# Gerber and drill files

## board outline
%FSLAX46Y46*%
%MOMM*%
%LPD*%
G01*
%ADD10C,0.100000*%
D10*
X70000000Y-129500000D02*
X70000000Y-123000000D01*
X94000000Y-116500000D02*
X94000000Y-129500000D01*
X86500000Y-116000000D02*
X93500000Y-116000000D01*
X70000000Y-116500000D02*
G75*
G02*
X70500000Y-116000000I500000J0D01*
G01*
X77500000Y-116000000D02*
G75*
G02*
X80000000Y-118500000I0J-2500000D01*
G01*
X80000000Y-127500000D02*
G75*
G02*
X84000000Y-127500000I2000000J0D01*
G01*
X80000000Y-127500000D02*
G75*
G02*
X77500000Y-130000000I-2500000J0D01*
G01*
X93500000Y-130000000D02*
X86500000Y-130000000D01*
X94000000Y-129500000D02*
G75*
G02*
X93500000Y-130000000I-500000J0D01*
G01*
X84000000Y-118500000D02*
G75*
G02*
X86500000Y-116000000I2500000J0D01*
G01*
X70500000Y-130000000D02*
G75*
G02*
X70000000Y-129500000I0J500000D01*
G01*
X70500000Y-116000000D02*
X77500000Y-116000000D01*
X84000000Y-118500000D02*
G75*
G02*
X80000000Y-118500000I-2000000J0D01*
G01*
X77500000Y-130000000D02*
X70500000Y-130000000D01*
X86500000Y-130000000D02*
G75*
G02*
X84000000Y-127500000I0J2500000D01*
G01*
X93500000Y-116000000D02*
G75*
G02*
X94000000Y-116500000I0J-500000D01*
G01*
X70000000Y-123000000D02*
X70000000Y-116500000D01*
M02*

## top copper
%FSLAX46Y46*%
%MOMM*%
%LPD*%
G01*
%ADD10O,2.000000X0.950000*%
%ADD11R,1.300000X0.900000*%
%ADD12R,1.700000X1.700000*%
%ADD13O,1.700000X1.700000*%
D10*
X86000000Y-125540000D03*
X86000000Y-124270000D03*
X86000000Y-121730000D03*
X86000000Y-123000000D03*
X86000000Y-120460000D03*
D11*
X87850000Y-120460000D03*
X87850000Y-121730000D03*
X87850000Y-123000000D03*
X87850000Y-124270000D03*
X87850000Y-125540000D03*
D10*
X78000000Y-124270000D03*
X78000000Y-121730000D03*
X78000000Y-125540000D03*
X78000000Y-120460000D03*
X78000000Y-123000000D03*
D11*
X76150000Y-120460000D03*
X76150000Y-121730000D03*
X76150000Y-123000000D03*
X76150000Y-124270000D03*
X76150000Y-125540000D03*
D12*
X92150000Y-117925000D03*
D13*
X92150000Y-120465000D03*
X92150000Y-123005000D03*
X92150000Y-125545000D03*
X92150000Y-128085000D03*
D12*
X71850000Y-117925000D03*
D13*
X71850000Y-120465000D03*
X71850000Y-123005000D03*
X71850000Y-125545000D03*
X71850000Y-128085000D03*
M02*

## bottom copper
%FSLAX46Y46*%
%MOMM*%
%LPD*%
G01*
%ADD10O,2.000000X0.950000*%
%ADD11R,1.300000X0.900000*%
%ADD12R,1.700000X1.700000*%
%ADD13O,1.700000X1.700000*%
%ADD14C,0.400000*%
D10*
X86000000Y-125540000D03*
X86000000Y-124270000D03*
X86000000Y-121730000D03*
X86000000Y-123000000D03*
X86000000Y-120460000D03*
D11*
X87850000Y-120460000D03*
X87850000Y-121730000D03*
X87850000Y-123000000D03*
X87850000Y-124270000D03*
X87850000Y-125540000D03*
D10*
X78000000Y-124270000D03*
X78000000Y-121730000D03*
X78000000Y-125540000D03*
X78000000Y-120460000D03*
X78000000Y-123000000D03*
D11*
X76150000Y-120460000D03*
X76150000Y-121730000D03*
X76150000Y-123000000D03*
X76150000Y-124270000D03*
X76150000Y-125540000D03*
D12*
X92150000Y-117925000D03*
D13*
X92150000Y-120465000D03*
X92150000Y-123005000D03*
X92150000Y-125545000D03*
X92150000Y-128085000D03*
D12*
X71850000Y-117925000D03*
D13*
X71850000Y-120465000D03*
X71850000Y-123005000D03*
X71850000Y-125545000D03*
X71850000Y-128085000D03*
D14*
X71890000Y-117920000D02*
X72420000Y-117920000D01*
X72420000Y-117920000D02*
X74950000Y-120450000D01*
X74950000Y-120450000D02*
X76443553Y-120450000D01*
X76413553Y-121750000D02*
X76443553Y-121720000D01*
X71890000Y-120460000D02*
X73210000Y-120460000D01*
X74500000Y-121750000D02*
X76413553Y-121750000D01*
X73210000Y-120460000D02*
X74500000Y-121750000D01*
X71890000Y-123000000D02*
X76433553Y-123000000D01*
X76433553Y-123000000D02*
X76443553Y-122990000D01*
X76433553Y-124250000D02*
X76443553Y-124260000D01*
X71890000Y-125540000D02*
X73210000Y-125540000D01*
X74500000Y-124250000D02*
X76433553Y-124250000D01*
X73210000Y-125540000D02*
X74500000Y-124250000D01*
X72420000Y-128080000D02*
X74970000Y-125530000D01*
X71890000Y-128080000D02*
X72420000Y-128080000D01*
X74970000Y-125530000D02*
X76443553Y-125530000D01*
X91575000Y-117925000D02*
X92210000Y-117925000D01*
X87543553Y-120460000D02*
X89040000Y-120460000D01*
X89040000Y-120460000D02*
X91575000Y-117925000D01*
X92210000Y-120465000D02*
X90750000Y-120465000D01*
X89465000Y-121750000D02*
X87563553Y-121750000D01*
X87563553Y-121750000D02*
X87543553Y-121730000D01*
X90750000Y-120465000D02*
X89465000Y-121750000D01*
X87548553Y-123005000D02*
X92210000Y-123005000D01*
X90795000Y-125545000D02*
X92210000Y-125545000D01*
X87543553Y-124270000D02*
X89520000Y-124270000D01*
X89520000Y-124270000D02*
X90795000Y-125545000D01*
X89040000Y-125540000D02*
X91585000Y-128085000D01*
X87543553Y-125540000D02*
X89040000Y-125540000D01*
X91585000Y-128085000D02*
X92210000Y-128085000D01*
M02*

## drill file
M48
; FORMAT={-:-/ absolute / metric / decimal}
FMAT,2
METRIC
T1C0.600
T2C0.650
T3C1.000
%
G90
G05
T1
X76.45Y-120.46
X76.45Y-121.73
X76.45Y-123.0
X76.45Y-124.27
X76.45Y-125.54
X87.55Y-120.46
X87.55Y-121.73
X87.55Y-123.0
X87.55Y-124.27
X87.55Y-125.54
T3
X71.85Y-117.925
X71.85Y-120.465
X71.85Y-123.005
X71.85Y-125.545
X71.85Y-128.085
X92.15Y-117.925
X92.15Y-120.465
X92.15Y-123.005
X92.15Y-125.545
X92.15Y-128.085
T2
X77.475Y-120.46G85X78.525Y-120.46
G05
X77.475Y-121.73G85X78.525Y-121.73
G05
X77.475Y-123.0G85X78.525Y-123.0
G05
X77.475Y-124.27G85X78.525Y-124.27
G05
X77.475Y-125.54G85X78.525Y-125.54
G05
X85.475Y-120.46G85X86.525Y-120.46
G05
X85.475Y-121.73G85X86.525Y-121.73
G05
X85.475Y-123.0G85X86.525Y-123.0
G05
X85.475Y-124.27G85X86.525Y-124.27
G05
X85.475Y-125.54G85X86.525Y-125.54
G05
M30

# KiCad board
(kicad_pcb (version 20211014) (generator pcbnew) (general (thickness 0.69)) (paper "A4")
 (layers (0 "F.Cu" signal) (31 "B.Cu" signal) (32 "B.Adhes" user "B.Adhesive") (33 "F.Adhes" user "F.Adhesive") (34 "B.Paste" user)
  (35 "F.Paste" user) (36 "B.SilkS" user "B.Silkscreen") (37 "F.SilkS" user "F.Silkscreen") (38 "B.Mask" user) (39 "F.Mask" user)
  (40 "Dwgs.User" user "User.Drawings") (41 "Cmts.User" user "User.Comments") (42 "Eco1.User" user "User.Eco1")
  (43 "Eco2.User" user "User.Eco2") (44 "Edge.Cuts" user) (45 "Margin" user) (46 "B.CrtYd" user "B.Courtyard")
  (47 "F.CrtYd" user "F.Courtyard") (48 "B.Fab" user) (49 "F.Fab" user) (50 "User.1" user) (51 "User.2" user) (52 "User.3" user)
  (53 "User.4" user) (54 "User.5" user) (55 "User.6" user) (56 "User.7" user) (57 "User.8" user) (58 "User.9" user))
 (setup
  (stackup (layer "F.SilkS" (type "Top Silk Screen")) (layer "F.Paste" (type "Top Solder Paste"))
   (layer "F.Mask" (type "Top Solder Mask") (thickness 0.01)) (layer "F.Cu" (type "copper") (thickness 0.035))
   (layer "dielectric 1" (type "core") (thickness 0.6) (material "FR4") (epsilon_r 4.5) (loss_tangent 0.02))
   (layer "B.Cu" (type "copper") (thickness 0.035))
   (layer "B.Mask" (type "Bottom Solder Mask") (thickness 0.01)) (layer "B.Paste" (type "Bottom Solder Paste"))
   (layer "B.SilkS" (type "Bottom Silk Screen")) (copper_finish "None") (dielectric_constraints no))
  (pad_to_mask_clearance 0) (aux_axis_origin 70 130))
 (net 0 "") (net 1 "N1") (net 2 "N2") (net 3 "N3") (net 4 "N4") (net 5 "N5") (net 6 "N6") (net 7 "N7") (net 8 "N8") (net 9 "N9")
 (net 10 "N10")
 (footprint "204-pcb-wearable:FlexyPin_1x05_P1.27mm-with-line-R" (layer "F.Cu") (at 86.05 120.46)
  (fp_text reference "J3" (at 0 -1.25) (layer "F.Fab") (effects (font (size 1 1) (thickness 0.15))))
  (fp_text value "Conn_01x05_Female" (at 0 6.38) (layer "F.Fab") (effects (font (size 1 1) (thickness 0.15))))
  (pad "" thru_hole oval (at -0.05 5.08) (size 2 0.95) (drill oval 1.7 0.65) (layers *.Cu *.Mask))
  (pad "" thru_hole oval (at -0.05 3.81) (size 2 0.95) (drill oval 1.7 0.65) (layers *.Cu *.Mask))
  (pad "" thru_hole oval (at -0.05 1.27) (size 2 0.95) (drill oval 1.7 0.65) (layers *.Cu *.Mask))
  (pad "" thru_hole oval (at -0.05 2.54) (size 2 0.95) (drill oval 1.7 0.65) (layers *.Cu *.Mask))
  (pad "" thru_hole oval (at -0.05 0) (size 2 0.95) (drill oval 1.7 0.65) (layers *.Cu *.Mask))
  (pad "1" thru_hole rect (at 1.5 0) (size 1.3 0.9) (drill 0.6 (offset 0.3 0)) (layers *.Cu *.Mask) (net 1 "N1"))
  (pad "2" thru_hole rect (at 1.5 1.27) (size 1.3 0.9) (drill 0.6 (offset 0.3 0)) (layers *.Cu *.Mask) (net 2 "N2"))
  (pad "3" thru_hole rect (at 1.5 2.54) (size 1.3 0.9) (drill 0.6 (offset 0.3 0)) (layers *.Cu *.Mask) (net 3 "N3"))
  (pad "4" thru_hole rect (at 1.5 3.81) (size 1.3 0.9) (drill 0.6 (offset 0.3 0)) (layers *.Cu *.Mask) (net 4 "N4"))
  (pad "5" thru_hole rect (at 1.5 5.08) (size 1.3 0.9) (drill 0.6 (offset 0.3 0)) (layers *.Cu *.Mask) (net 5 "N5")))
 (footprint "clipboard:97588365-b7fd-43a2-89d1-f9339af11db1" (layer "F.Cu") (at 85.499999 126.499999 180)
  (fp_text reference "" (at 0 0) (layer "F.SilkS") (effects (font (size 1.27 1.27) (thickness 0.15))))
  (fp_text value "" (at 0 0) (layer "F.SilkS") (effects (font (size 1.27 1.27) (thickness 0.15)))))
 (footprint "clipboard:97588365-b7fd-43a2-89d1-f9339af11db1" (layer "F.Cu") (at 78.500001 126.499999 90)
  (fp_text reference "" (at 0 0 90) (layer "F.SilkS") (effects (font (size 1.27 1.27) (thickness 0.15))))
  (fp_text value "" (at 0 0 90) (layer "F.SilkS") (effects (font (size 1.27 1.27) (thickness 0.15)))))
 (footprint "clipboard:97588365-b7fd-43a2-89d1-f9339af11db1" (layer "F.Cu") (at 85.499999 119.500001 -90)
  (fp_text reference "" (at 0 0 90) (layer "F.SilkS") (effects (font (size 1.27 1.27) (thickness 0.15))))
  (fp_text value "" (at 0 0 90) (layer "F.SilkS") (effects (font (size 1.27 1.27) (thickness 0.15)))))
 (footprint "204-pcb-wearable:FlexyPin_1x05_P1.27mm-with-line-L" (layer "F.Cu") (at 76.45 120.46)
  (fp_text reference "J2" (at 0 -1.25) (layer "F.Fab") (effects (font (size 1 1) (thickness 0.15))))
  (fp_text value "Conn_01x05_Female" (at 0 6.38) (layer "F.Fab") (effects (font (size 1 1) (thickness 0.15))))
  (pad "" thru_hole oval (at 1.55 3.81) (size 2 0.95) (drill oval 1.7 0.65) (layers *.Cu *.Mask))
  (pad "" thru_hole oval (at 1.55 1.27) (size 2 0.95) (drill oval 1.7 0.65) (layers *.Cu *.Mask))
  (pad "" thru_hole oval (at 1.55 5.08) (size 2 0.95) (drill oval 1.7 0.65) (layers *.Cu *.Mask))
  (pad "" thru_hole oval (at 1.55 0) (size 2 0.95) (drill oval 1.7 0.65) (layers *.Cu *.Mask))
  (pad "" thru_hole oval (at 1.55 2.54) (size 2 0.95) (drill oval 1.7 0.65) (layers *.Cu *.Mask))
  (pad "1" thru_hole rect (at 0 0) (size 1.3 0.9) (drill 0.6 (offset -0.3 0)) (layers *.Cu *.Mask) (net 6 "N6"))
  (pad "2" thru_hole rect (at 0 1.27) (size 1.3 0.9) (drill 0.6 (offset -0.3 0)) (layers *.Cu *.Mask) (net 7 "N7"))
  (pad "3" thru_hole rect (at 0 2.54) (size 1.3 0.9) (drill 0.6 (offset -0.3 0)) (layers *.Cu *.Mask) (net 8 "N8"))
  (pad "4" thru_hole rect (at 0 3.81) (size 1.3 0.9) (drill 0.6 (offset -0.3 0)) (layers *.Cu *.Mask) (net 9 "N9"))
  (pad "5" thru_hole rect (at 0 5.08) (size 1.3 0.9) (drill 0.6 (offset -0.3 0)) (layers *.Cu *.Mask) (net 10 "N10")))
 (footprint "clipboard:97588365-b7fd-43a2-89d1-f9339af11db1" (layer "F.Cu") (at 78.500001 119.500001)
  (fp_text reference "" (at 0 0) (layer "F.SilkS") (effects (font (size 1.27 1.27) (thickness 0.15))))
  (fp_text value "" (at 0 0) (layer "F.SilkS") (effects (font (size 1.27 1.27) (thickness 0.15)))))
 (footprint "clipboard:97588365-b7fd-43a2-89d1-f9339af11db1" (layer "B.Cu") (at 78.500001 119.500001 -90)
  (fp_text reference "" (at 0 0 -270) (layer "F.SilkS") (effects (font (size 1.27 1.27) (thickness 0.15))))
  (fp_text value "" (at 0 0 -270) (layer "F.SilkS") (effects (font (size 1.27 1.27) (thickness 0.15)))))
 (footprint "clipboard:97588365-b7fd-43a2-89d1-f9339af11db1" (layer "B.Cu") (at 78.500001 126.499999)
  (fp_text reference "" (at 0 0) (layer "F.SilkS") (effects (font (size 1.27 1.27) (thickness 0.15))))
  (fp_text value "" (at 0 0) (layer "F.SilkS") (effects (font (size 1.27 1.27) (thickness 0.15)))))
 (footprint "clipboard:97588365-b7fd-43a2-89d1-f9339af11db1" (layer "B.Cu") (at 85.499999 119.500001 180)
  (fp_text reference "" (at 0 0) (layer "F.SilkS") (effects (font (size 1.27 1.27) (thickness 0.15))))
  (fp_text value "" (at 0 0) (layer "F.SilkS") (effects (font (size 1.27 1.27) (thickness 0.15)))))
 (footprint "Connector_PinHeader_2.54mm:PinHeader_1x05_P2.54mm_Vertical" (layer "B.Cu") (at 92.15 117.925 180)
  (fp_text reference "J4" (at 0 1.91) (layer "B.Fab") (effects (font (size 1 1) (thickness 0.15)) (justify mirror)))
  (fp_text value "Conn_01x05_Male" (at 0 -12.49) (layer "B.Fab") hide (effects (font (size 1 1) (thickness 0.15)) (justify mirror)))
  (pad "1" thru_hole rect (at 0 0 180) (size 1.7 1.7) (drill 1) (layers *.Cu *.Mask) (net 1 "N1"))
  (pad "2" thru_hole oval (at 0 -2.54 180) (size 1.7 1.7) (drill 1) (layers *.Cu *.Mask) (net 2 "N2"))
  (pad "3" thru_hole oval (at 0 -5.08 180) (size 1.7 1.7) (drill 1) (layers *.Cu *.Mask) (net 3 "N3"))
  (pad "4" thru_hole oval (at 0 -7.62 180) (size 1.7 1.7) (drill 1) (layers *.Cu *.Mask) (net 4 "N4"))
  (pad "5" thru_hole oval (at 0 -10.16 180) (size 1.7 1.7) (drill 1) (layers *.Cu *.Mask) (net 5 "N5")))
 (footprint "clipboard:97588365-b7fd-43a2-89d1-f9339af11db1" (layer "B.Cu") (at 85.499999 126.499999 90)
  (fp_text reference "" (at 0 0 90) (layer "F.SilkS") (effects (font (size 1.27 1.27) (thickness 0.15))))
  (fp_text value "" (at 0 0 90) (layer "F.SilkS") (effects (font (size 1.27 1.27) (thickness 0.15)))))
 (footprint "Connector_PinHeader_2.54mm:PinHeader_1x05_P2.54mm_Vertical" (layer "B.Cu") (at 71.85 117.925 180)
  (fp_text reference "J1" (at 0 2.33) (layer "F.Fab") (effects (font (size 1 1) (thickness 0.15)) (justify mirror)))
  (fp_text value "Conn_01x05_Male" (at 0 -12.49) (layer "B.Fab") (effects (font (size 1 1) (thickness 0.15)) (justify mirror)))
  (pad "1" thru_hole rect (at 0 0 180) (size 1.7 1.7) (drill 1) (layers *.Cu *.Mask) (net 6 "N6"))
  (pad "2" thru_hole oval (at 0 -2.54 180) (size 1.7 1.7) (drill 1) (layers *.Cu *.Mask) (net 7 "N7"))
  (pad "3" thru_hole oval (at 0 -5.08 180) (size 1.7 1.7) (drill 1) (layers *.Cu *.Mask) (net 8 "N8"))
  (pad "4" thru_hole oval (at 0 -7.62 180) (size 1.7 1.7) (drill 1) (layers *.Cu *.Mask) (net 9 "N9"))
  (pad "5" thru_hole oval (at 0 -10.16 180) (size 1.7 1.7) (drill 1) (layers *.Cu *.Mask) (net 10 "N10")))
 (gr_line (start 70 129.5) (end 70 123) (layer "Edge.Cuts") (width 0.1))
 (gr_line (start 94 116.5) (end 94 129.5) (layer "Edge.Cuts") (width 0.1))
 (gr_line (start 86.5 116) (end 93.5 116) (layer "Edge.Cuts") (width 0.1))
 (gr_arc (start 70 116.5) (mid 70.146447 116.146447) (end 70.5 116) (layer "Edge.Cuts") (width 0.1))
 (gr_arc (start 77.5 116) (mid 79.267767 116.732233) (end 80 118.5) (layer "Edge.Cuts") (width 0.1))
 (gr_arc (start 80 127.5) (mid 82 125.5) (end 84 127.5) (layer "Edge.Cuts") (width 0.1))
 (gr_arc (start 80 127.5) (mid 79.267767 129.267767) (end 77.5 130) (layer "Edge.Cuts") (width 0.1))
 (gr_line (start 93.5 130) (end 86.5 130) (layer "Edge.Cuts") (width 0.1))
 (gr_arc (start 94 129.5) (mid 93.853553 129.853553) (end 93.5 130) (layer "Edge.Cuts") (width 0.1))
 (gr_arc (start 84 118.5) (mid 84.732233 116.732233) (end 86.5 116) (layer "Edge.Cuts") (width 0.1))
 (gr_arc (start 70.5 130) (mid 70.146447 129.853553) (end 70 129.5) (layer "Edge.Cuts") (width 0.1))
 (gr_line (start 70.5 116) (end 77.5 116) (layer "Edge.Cuts") (width 0.1))
 (gr_arc (start 84 118.5) (mid 82 120.5) (end 80 118.5) (layer "Edge.Cuts") (width 0.1))
 (gr_line (start 77.5 130) (end 70.5 130) (layer "Edge.Cuts") (width 0.1))
 (gr_arc (start 86.5 130) (mid 84.732233 129.267767) (end 84 127.5) (layer "Edge.Cuts") (width 0.1))
 (gr_arc (start 93.5 116) (mid 93.853553 116.146447) (end 94 116.5) (layer "Edge.Cuts") (width 0.1))
 (gr_line (start 70 123) (end 70 116.5) (layer "Edge.Cuts") (width 0.1))
 (segment (start 71.89 117.92) (end 72.42 117.92) (width 0.4) (layer "B.Cu") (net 6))
 (segment (start 72.42 117.92) (end 74.95 120.45) (width 0.4) (layer "B.Cu") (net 6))
 (segment (start 74.95 120.45) (end 76.443553 120.45) (width 0.4) (layer "B.Cu") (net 6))
 (segment (start 76.413553 121.75) (end 76.443553 121.72) (width 0.4) (layer "B.Cu") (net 7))
 (segment (start 71.89 120.46) (end 73.21 120.46) (width 0.4) (layer "B.Cu") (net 7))
 (segment (start 74.5 121.75) (end 76.413553 121.75) (width 0.4) (layer "B.Cu") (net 7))
 (segment (start 73.21 120.46) (end 74.5 121.75) (width 0.4) (layer "B.Cu") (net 7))
 (segment (start 71.89 123) (end 76.433553 123) (width 0.4) (layer "B.Cu") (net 8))
 (segment (start 76.433553 123) (end 76.443553 122.99) (width 0.4) (layer "B.Cu") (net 8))
 (segment (start 76.433553 124.25) (end 76.443553 124.26) (width 0.4) (layer "B.Cu") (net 9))
 (segment (start 71.89 125.54) (end 73.21 125.54) (width 0.4) (layer "B.Cu") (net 9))
 (segment (start 74.5 124.25) (end 76.433553 124.25) (width 0.4) (layer "B.Cu") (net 9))
 (segment (start 73.21 125.54) (end 74.5 124.25) (width 0.4) (layer "B.Cu") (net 9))
 (segment (start 72.42 128.08) (end 74.97 125.53) (width 0.4) (layer "B.Cu") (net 10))
 (segment (start 71.89 128.08) (end 72.42 128.08) (width 0.4) (layer "B.Cu") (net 10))
 (segment (start 74.97 125.53) (end 76.443553 125.53) (width 0.4) (layer "B.Cu") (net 10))
 (segment (start 91.575 117.925) (end 92.21 117.925) (width 0.4) (layer "B.Cu") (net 1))
 (segment (start 87.543553 120.46) (end 89.04 120.46) (width 0.4) (layer "B.Cu") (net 1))
 (segment (start 89.04 120.46) (end 91.575 117.925) (width 0.4) (layer "B.Cu") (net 1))
 (segment (start 92.21 120.465) (end 90.75 120.465) (width 0.4) (layer "B.Cu") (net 2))
 (segment (start 89.465 121.75) (end 87.563553 121.75) (width 0.4) (layer "B.Cu") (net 2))
 (segment (start 87.563553 121.75) (end 87.543553 121.73) (width 0.4) (layer "B.Cu") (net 2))
 (segment (start 90.75 120.465) (end 89.465 121.75) (width 0.4) (layer "B.Cu") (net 2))
 (segment (start 87.548553 123.005) (end 92.21 123.005) (width 0.4) (layer "B.Cu") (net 3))
 (segment (start 90.795 125.545) (end 92.21 125.545) (width 0.4) (layer "B.Cu") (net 4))
 (segment (start 87.543553 124.27) (end 89.52 124.27) (width 0.4) (layer "B.Cu") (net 4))
 (segment (start 89.52 124.27) (end 90.795 125.545) (width 0.4) (layer "B.Cu") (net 4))
 (segment (start 89.04 125.54) (end 91.585 128.085) (width 0.4) (layer "B.Cu") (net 5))
 (segment (start 87.543553 125.54) (end 89.04 125.54) (width 0.4) (layer "B.Cu") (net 5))
 (segment (start 91.585 128.085) (end 92.21 128.085) (width 0.4) (layer "B.Cu") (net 5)))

